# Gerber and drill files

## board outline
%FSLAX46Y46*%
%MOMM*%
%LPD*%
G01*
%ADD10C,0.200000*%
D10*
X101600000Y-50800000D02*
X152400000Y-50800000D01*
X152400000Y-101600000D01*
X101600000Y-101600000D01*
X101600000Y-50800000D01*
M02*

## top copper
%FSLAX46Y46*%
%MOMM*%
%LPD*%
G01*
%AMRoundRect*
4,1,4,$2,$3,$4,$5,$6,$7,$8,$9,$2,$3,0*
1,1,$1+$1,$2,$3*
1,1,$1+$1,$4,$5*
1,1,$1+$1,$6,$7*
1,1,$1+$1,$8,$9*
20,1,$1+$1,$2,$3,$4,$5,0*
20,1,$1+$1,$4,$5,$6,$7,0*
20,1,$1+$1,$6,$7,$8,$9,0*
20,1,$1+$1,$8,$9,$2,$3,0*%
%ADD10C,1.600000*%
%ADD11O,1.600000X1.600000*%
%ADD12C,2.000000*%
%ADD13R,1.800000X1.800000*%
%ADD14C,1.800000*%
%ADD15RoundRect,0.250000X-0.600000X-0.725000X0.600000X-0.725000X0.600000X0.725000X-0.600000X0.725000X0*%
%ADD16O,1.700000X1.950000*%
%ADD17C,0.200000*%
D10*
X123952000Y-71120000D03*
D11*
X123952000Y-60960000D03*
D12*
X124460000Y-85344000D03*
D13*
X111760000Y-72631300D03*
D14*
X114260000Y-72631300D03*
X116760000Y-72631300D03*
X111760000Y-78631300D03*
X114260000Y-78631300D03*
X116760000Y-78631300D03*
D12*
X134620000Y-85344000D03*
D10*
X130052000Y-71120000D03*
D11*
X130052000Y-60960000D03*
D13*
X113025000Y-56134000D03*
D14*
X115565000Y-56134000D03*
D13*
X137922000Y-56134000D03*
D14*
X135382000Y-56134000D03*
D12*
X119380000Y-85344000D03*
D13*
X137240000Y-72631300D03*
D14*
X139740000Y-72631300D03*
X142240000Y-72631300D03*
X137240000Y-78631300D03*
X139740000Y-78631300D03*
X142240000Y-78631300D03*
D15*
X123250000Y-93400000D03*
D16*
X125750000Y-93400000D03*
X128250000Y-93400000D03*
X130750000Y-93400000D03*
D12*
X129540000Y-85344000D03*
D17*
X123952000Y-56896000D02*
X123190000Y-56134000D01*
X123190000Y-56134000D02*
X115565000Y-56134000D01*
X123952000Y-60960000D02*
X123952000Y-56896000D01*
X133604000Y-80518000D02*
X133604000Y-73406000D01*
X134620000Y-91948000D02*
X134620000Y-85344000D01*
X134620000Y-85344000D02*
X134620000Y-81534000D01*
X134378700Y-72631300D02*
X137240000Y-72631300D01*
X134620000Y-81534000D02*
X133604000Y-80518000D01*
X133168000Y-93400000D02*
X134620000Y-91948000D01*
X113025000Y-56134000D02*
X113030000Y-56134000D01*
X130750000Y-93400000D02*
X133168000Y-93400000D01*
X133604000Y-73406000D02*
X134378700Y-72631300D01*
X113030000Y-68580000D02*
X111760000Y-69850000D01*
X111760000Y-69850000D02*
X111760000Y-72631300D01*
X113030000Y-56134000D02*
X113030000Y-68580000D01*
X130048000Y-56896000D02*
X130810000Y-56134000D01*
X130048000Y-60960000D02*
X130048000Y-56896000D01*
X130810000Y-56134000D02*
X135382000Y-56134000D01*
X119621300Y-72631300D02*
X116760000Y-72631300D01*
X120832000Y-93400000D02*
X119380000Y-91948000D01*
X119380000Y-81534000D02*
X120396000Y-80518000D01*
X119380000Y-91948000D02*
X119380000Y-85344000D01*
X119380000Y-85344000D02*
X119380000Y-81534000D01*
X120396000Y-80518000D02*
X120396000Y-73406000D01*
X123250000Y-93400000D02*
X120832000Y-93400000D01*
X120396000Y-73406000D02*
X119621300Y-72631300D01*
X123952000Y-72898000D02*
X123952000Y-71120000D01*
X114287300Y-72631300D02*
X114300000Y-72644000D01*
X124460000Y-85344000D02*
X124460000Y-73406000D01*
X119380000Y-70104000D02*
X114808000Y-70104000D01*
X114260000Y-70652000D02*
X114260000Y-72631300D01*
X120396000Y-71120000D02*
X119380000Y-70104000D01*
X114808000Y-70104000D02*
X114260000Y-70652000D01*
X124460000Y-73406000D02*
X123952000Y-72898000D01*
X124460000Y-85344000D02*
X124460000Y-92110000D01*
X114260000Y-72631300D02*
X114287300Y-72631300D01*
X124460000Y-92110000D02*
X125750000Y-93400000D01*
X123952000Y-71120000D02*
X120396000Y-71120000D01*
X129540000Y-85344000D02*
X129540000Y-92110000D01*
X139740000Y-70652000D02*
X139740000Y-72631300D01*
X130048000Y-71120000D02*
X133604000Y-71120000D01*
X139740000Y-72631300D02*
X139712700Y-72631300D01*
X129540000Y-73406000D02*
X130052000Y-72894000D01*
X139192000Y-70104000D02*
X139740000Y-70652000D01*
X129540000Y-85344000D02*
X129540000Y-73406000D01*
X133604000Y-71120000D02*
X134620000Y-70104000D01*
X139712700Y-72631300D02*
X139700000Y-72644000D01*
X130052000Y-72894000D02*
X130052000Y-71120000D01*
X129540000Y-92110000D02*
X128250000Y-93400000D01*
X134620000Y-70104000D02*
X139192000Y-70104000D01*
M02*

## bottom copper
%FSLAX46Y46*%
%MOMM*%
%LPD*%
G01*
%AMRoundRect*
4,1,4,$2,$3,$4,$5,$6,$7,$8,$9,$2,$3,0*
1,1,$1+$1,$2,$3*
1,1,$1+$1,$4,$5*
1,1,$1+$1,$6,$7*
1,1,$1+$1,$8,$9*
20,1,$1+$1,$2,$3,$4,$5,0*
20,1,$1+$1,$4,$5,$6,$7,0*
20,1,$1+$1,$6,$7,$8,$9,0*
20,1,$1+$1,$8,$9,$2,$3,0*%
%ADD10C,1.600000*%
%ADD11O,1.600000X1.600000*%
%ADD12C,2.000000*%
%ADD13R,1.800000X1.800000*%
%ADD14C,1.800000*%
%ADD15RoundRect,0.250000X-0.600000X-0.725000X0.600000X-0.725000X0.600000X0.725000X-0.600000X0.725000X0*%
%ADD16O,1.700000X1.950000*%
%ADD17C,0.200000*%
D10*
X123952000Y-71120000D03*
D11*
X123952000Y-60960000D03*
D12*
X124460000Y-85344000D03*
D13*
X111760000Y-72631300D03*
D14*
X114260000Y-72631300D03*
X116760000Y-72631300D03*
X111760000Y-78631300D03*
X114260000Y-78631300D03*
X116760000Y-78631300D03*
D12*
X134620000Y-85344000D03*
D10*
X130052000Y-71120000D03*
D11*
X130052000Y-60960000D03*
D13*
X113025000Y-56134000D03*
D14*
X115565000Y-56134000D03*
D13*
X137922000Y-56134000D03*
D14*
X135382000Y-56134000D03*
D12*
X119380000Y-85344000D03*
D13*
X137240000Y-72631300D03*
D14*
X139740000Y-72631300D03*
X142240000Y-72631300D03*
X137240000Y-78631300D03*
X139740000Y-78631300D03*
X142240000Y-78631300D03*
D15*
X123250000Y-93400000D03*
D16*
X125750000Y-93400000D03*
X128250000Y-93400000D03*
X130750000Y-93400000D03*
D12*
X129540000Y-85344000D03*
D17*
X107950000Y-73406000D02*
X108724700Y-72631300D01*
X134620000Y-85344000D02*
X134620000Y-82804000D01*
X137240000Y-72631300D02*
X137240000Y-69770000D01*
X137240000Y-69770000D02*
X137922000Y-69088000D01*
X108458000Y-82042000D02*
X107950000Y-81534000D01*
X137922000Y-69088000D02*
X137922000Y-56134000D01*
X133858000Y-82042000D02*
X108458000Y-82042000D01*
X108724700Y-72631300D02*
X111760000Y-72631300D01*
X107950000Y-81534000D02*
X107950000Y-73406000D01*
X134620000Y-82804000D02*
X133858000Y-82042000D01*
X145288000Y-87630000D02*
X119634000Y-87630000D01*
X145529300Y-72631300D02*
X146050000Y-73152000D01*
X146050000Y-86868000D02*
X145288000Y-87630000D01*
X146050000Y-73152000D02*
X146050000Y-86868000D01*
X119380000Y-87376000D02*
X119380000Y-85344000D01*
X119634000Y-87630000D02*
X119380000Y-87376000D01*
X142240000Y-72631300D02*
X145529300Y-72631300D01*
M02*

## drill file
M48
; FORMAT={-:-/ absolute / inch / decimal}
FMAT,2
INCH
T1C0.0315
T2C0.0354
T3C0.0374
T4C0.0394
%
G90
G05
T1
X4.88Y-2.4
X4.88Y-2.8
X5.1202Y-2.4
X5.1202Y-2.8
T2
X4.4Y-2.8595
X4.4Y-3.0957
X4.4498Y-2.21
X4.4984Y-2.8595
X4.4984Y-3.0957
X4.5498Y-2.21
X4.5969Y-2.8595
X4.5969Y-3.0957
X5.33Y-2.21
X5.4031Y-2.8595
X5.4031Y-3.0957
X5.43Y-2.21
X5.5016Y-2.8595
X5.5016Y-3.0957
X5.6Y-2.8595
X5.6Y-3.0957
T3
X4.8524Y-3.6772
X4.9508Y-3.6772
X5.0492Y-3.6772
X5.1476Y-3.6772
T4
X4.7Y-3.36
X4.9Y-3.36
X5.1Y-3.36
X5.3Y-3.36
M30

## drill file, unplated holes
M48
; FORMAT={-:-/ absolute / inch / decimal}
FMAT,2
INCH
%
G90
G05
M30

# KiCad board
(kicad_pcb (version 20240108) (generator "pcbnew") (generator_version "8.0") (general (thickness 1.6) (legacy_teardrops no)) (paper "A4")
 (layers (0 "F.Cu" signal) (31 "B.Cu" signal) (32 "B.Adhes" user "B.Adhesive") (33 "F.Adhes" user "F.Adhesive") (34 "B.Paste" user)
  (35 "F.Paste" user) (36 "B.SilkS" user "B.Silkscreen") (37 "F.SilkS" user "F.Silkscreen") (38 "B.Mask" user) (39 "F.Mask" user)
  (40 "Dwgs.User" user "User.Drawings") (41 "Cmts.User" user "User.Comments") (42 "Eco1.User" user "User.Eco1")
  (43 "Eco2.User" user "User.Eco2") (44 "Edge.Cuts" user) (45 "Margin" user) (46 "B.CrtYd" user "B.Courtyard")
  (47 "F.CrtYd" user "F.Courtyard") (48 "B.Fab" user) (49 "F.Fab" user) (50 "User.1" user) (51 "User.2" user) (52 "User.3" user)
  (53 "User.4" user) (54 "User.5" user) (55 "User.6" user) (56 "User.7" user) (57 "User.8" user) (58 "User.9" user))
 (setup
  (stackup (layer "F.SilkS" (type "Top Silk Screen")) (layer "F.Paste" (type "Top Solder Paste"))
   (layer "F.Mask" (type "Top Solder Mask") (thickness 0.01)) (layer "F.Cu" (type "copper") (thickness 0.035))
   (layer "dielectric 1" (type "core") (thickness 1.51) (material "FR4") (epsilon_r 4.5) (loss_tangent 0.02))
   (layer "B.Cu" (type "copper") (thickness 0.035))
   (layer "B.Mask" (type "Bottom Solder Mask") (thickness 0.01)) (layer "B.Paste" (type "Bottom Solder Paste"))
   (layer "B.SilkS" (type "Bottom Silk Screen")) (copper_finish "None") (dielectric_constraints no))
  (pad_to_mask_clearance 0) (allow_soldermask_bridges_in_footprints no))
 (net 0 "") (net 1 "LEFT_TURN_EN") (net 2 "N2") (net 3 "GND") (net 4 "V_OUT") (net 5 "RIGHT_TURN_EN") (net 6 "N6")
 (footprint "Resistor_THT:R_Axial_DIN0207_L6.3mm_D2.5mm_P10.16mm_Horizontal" (layer "F.Cu") (at 123.952 71.12 90)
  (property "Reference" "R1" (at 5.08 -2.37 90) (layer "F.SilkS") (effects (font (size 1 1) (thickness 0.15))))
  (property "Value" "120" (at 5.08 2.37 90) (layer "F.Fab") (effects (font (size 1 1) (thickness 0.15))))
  (pad "1" thru_hole circle (at 0 0 90) (size 1.6 1.6) (drill 0.8) (layers "*.Cu" "*.Mask") (remove_unused_layers no) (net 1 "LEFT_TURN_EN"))
  (pad "2" thru_hole oval (at 10.16 0 90) (size 1.6 1.6) (drill 0.8) (layers "*.Cu" "*.Mask") (remove_unused_layers no) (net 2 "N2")))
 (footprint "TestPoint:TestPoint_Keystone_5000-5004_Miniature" (layer "F.Cu") (at 124.46 85.344)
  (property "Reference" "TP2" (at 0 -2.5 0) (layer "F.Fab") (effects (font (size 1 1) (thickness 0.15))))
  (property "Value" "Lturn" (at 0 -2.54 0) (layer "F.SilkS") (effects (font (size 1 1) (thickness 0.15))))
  (pad "1" thru_hole circle (at 0 0) (size 2 2) (drill 1) (layers "*.Cu" "*.Mask") (remove_unused_layers no) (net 1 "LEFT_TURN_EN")))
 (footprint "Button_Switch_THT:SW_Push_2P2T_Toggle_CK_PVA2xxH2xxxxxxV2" (layer "F.Cu") (at 111.76 72.6313)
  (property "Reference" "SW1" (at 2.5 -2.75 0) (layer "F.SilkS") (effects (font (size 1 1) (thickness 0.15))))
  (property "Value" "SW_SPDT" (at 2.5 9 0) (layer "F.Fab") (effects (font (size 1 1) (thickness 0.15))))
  (pad "1" thru_hole rect (at 0 0) (size 1.8 1.8) (drill 0.9) (layers "*.Cu" "*.Mask") (remove_unused_layers no) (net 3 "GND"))
  (pad "2" thru_hole circle (at 2.5 0) (size 1.8 1.8) (drill 0.9) (layers "*.Cu" "*.Mask") (remove_unused_layers no) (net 1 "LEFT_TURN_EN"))
  (pad "3" thru_hole circle (at 5 0) (size 1.8 1.8) (drill 0.9) (layers "*.Cu" "*.Mask") (remove_unused_layers no) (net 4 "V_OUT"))
  (pad "4" thru_hole circle (at 0 6) (size 1.8 1.8) (drill 0.9) (layers "*.Cu" "*.Mask") (remove_unused_layers no))
  (pad "5" thru_hole circle (at 2.5 6) (size 1.8 1.8) (drill 0.9) (layers "*.Cu" "*.Mask") (remove_unused_layers no))
  (pad "6" thru_hole circle (at 5 6) (size 1.8 1.8) (drill 0.9) (layers "*.Cu" "*.Mask") (remove_unused_layers no)))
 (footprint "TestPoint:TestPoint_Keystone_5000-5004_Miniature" (layer "F.Cu") (at 134.62 85.344)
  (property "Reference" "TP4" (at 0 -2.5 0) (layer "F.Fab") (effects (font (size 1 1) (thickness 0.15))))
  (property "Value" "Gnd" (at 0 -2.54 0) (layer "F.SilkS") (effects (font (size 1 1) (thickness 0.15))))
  (pad "1" thru_hole circle (at 0 0) (size 2 2) (drill 1) (layers "*.Cu" "*.Mask") (remove_unused_layers no) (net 3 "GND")))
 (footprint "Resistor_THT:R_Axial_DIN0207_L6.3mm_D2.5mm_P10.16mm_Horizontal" (layer "F.Cu") (at 130.052 71.12 90)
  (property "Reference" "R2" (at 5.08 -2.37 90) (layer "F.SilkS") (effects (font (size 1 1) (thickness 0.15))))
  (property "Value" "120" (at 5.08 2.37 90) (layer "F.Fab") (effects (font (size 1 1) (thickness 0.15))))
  (pad "1" thru_hole circle (at 0 0 90) (size 1.6 1.6) (drill 0.8) (layers "*.Cu" "*.Mask") (remove_unused_layers no)
   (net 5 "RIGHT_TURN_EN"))
  (pad "2" thru_hole oval (at 10.16 0 90) (size 1.6 1.6) (drill 0.8) (layers "*.Cu" "*.Mask") (remove_unused_layers no) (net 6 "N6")))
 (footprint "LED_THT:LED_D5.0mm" (layer "F.Cu") (at 113.025 56.134)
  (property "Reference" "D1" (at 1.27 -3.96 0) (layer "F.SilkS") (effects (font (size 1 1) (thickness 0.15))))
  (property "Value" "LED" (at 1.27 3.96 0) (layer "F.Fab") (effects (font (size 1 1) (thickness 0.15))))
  (pad "1" thru_hole rect (at 0 0) (size 1.8 1.8) (drill 0.9) (layers "*.Cu" "*.Mask") (remove_unused_layers no) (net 3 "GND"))
  (pad "2" thru_hole circle (at 2.54 0) (size 1.8 1.8) (drill 0.9) (layers "*.Cu" "*.Mask") (remove_unused_layers no) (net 2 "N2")))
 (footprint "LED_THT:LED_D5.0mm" (layer "F.Cu") (at 137.922 56.134 180)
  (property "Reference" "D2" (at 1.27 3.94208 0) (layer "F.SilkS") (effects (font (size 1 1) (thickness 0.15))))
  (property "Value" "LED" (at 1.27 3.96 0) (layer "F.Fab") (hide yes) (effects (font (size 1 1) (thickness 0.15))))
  (pad "1" thru_hole rect (at 0 0 180) (size 1.8 1.8) (drill 0.9) (layers "*.Cu" "*.Mask") (remove_unused_layers no) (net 3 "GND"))
  (pad "2" thru_hole circle (at 2.54 0 180) (size 1.8 1.8) (drill 0.9) (layers "*.Cu" "*.Mask") (remove_unused_layers no) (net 6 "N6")))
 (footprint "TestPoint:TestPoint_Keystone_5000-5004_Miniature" (layer "F.Cu") (at 119.38 85.344)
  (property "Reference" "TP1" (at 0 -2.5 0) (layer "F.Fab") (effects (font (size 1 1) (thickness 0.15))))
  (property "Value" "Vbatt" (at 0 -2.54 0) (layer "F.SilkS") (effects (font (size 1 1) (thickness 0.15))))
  (pad "1" thru_hole circle (at 0 0) (size 2 2) (drill 1) (layers "*.Cu" "*.Mask") (remove_unused_layers no) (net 4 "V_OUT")))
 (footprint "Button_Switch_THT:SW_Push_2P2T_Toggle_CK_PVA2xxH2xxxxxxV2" (layer "F.Cu") (at 137.24 72.6313)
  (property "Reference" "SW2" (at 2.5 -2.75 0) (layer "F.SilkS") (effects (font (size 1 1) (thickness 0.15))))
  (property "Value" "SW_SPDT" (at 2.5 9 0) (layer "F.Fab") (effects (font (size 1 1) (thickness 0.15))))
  (pad "1" thru_hole rect (at 0 0) (size 1.8 1.8) (drill 0.9) (layers "*.Cu" "*.Mask") (remove_unused_layers no) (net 3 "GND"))
  (pad "2" thru_hole circle (at 2.5 0) (size 1.8 1.8) (drill 0.9) (layers "*.Cu" "*.Mask") (remove_unused_layers no) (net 5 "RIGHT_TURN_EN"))
  (pad "3" thru_hole circle (at 5 0) (size 1.8 1.8) (drill 0.9) (layers "*.Cu" "*.Mask") (remove_unused_layers no) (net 4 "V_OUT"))
  (pad "4" thru_hole circle (at 0 6) (size 1.8 1.8) (drill 0.9) (layers "*.Cu" "*.Mask") (remove_unused_layers no))
  (pad "5" thru_hole circle (at 2.5 6) (size 1.8 1.8) (drill 0.9) (layers "*.Cu" "*.Mask") (remove_unused_layers no))
  (pad "6" thru_hole circle (at 5 6) (size 1.8 1.8) (drill 0.9) (layers "*.Cu" "*.Mask") (remove_unused_layers no)))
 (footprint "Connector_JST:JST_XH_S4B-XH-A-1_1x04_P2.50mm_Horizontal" (layer "F.Cu") (at 123.25 93.4)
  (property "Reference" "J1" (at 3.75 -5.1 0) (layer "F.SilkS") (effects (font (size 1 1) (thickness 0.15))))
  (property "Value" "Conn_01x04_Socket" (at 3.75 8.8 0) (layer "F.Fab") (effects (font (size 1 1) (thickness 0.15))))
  (pad "1" thru_hole roundrect (at 0 0) (size 1.7 1.95) (drill 0.95) (layers "*.Cu" "*.Mask") (remove_unused_layers no)
   (roundrect_rratio 0.147059) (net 4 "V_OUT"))
  (pad "2" thru_hole oval (at 2.5 0) (size 1.7 1.95) (drill 0.95) (layers "*.Cu" "*.Mask") (remove_unused_layers no) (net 1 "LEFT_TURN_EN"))
  (pad "3" thru_hole oval (at 5 0) (size 1.7 1.95) (drill 0.95) (layers "*.Cu" "*.Mask") (remove_unused_layers no) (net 5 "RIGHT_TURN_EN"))
  (pad "4" thru_hole oval (at 7.5 0) (size 1.7 1.95) (drill 0.95) (layers "*.Cu" "*.Mask") (remove_unused_layers no) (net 3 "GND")))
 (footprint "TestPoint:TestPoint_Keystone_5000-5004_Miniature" (layer "F.Cu") (at 129.54 85.344)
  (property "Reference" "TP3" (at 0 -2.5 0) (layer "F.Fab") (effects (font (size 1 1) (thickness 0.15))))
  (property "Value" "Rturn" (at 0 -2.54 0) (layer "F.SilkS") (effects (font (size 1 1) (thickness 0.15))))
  (pad "1" thru_hole circle (at 0 0) (size 2 2) (drill 1) (layers "*.Cu" "*.Mask") (remove_unused_layers no) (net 5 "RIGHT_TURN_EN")))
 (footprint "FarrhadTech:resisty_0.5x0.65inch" (layer "B.Cu") (at 145.034 93.98 180)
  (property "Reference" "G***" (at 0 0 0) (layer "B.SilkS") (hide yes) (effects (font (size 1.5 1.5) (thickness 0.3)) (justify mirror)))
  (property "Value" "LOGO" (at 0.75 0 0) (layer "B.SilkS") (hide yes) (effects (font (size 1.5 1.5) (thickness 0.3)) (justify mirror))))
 (gr_rect (start 101.6 50.8) (end 152.4 101.6) (stroke (width 0.2) (type default)) (fill none) (layer "Edge.Cuts"))
 (segment (start 123.952 56.896) (end 123.19 56.134) (width 0.2) (layer "F.Cu") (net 2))
 (segment (start 123.19 56.134) (end 115.565 56.134) (width 0.2) (layer "F.Cu") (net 2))
 (segment (start 123.952 60.96) (end 123.952 56.896) (width 0.2) (layer "F.Cu") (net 2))
 (segment (start 133.604 80.518) (end 133.604 73.406) (width 0.2) (layer "F.Cu") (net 3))
 (segment (start 134.62 91.948) (end 134.62 85.344) (width 0.2) (layer "F.Cu") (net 3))
 (segment (start 134.62 85.344) (end 134.62 81.534) (width 0.2) (layer "F.Cu") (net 3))
 (segment (start 134.3787 72.6313) (end 137.24 72.6313) (width 0.2) (layer "F.Cu") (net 3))
 (segment (start 134.62 81.534) (end 133.604 80.518) (width 0.2) (layer "F.Cu") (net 3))
 (segment (start 133.168 93.4) (end 134.62 91.948) (width 0.2) (layer "F.Cu") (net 3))
 (segment (start 113.025 56.134) (end 113.03 56.134) (width 0.2) (layer "F.Cu") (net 3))
 (segment (start 130.75 93.4) (end 133.168 93.4) (width 0.2) (layer "F.Cu") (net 3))
 (segment (start 133.604 73.406) (end 134.3787 72.6313) (width 0.2) (layer "F.Cu") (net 3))
 (segment (start 113.03 68.58) (end 111.76 69.85) (width 0.2) (layer "F.Cu") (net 3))
 (segment (start 111.76 69.85) (end 111.76 72.6313) (width 0.2) (layer "F.Cu") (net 3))
 (segment (start 113.03 56.134) (end 113.03 68.58) (width 0.2) (layer "F.Cu") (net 3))
 (segment (start 107.95 73.406) (end 108.7247 72.6313) (width 0.2) (layer "B.Cu") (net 3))
 (segment (start 134.62 85.344) (end 134.62 82.804) (width 0.2) (layer "B.Cu") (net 3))
 (segment (start 137.24 72.6313) (end 137.24 69.77) (width 0.2) (layer "B.Cu") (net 3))
 (segment (start 137.24 69.77) (end 137.922 69.088) (width 0.2) (layer "B.Cu") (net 3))
 (segment (start 108.458 82.042) (end 107.95 81.534) (width 0.2) (layer "B.Cu") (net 3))
 (segment (start 137.922 69.088) (end 137.922 56.134) (width 0.2) (layer "B.Cu") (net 3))
 (segment (start 133.858 82.042) (end 108.458 82.042) (width 0.2) (layer "B.Cu") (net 3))
 (segment (start 108.7247 72.6313) (end 111.76 72.6313) (width 0.2) (layer "B.Cu") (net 3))
 (segment (start 107.95 81.534) (end 107.95 73.406) (width 0.2) (layer "B.Cu") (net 3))
 (segment (start 134.62 82.804) (end 133.858 82.042) (width 0.2) (layer "B.Cu") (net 3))
 (segment (start 130.048 56.896) (end 130.81 56.134) (width 0.2) (layer "F.Cu") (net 6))
 (segment (start 130.048 60.96) (end 130.048 56.896) (width 0.2) (layer "F.Cu") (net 6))
 (segment (start 130.81 56.134) (end 135.382 56.134) (width 0.2) (layer "F.Cu") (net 6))
 (segment (start 119.6213 72.6313) (end 116.76 72.6313) (width 0.2) (layer "F.Cu") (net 4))
 (segment (start 120.832 93.4) (end 119.38 91.948) (width 0.2) (layer "F.Cu") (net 4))
 (segment (start 119.38 81.534) (end 120.396 80.518) (width 0.2) (layer "F.Cu") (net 4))
 (segment (start 119.38 91.948) (end 119.38 85.344) (width 0.2) (layer "F.Cu") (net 4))
 (segment (start 119.38 85.344) (end 119.38 81.534) (width 0.2) (layer "F.Cu") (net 4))
 (segment (start 120.396 80.518) (end 120.396 73.406) (width 0.2) (layer "F.Cu") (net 4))
 (segment (start 123.25 93.4) (end 120.832 93.4) (width 0.2) (layer "F.Cu") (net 4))
 (segment (start 120.396 73.406) (end 119.6213 72.6313) (width 0.2) (layer "F.Cu") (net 4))
 (segment (start 145.288 87.63) (end 119.634 87.63) (width 0.2) (layer "B.Cu") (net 4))
 (segment (start 145.5293 72.6313) (end 146.05 73.152) (width 0.2) (layer "B.Cu") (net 4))
 (segment (start 146.05 86.868) (end 145.288 87.63) (width 0.2) (layer "B.Cu") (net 4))
 (segment (start 146.05 73.152) (end 146.05 86.868) (width 0.2) (layer "B.Cu") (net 4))
 (segment (start 119.38 87.376) (end 119.38 85.344) (width 0.2) (layer "B.Cu") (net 4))
 (segment (start 119.634 87.63) (end 119.38 87.376) (width 0.2) (layer "B.Cu") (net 4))
 (segment (start 142.24 72.6313) (end 145.5293 72.6313) (width 0.2) (layer "B.Cu") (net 4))
 (segment (start 123.952 72.898) (end 123.952 71.12) (width 0.2) (layer "F.Cu") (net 1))
 (segment (start 114.2873 72.6313) (end 114.3 72.644) (width 0.2) (layer "F.Cu") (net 1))
 (segment (start 124.46 85.344) (end 124.46 73.406) (width 0.2) (layer "F.Cu") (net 1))
 (segment (start 119.38 70.104) (end 114.808 70.104) (width 0.2) (layer "F.Cu") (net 1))
 (segment (start 114.26 70.652) (end 114.26 72.6313) (width 0.2) (layer "F.Cu") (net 1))
 (segment (start 120.396 71.12) (end 119.38 70.104) (width 0.2) (layer "F.Cu") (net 1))
 (segment (start 114.808 70.104) (end 114.26 70.652) (width 0.2) (layer "F.Cu") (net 1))
 (segment (start 124.46 73.406) (end 123.952 72.898) (width 0.2) (layer "F.Cu") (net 1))
 (segment (start 124.46 85.344) (end 124.46 92.11) (width 0.2) (layer "F.Cu") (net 1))
 (segment (start 114.26 72.6313) (end 114.2873 72.6313) (width 0.2) (layer "F.Cu") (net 1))
 (segment (start 124.46 92.11) (end 125.75 93.4) (width 0.2) (layer "F.Cu") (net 1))
 (segment (start 123.952 71.12) (end 120.396 71.12) (width 0.2) (layer "F.Cu") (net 1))
 (segment (start 129.54 85.344) (end 129.54 92.11) (width 0.2) (layer "F.Cu") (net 5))
 (segment (start 139.74 70.652) (end 139.74 72.6313) (width 0.2) (layer "F.Cu") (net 5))
 (segment (start 130.048 71.12) (end 133.604 71.12) (width 0.2) (layer "F.Cu") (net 5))
 (segment (start 139.74 72.6313) (end 139.7127 72.6313) (width 0.2) (layer "F.Cu") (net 5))
 (segment (start 129.54 73.406) (end 130.052 72.894) (width 0.2) (layer "F.Cu") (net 5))
 (segment (start 139.192 70.104) (end 139.74 70.652) (width 0.2) (layer "F.Cu") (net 5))
 (segment (start 129.54 85.344) (end 129.54 73.406) (width 0.2) (layer "F.Cu") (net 5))
 (segment (start 133.604 71.12) (end 134.62 70.104) (width 0.2) (layer "F.Cu") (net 5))
 (segment (start 139.7127 72.6313) (end 139.7 72.644) (width 0.2) (layer "F.Cu") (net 5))
 (segment (start 130.052 72.894) (end 130.052 71.12) (width 0.2) (layer "F.Cu") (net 5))
 (segment (start 129.54 92.11) (end 128.25 93.4) (width 0.2) (layer "F.Cu") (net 5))
 (segment (start 134.62 70.104) (end 139.192 70.104) (width 0.2) (layer "F.Cu") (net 5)))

